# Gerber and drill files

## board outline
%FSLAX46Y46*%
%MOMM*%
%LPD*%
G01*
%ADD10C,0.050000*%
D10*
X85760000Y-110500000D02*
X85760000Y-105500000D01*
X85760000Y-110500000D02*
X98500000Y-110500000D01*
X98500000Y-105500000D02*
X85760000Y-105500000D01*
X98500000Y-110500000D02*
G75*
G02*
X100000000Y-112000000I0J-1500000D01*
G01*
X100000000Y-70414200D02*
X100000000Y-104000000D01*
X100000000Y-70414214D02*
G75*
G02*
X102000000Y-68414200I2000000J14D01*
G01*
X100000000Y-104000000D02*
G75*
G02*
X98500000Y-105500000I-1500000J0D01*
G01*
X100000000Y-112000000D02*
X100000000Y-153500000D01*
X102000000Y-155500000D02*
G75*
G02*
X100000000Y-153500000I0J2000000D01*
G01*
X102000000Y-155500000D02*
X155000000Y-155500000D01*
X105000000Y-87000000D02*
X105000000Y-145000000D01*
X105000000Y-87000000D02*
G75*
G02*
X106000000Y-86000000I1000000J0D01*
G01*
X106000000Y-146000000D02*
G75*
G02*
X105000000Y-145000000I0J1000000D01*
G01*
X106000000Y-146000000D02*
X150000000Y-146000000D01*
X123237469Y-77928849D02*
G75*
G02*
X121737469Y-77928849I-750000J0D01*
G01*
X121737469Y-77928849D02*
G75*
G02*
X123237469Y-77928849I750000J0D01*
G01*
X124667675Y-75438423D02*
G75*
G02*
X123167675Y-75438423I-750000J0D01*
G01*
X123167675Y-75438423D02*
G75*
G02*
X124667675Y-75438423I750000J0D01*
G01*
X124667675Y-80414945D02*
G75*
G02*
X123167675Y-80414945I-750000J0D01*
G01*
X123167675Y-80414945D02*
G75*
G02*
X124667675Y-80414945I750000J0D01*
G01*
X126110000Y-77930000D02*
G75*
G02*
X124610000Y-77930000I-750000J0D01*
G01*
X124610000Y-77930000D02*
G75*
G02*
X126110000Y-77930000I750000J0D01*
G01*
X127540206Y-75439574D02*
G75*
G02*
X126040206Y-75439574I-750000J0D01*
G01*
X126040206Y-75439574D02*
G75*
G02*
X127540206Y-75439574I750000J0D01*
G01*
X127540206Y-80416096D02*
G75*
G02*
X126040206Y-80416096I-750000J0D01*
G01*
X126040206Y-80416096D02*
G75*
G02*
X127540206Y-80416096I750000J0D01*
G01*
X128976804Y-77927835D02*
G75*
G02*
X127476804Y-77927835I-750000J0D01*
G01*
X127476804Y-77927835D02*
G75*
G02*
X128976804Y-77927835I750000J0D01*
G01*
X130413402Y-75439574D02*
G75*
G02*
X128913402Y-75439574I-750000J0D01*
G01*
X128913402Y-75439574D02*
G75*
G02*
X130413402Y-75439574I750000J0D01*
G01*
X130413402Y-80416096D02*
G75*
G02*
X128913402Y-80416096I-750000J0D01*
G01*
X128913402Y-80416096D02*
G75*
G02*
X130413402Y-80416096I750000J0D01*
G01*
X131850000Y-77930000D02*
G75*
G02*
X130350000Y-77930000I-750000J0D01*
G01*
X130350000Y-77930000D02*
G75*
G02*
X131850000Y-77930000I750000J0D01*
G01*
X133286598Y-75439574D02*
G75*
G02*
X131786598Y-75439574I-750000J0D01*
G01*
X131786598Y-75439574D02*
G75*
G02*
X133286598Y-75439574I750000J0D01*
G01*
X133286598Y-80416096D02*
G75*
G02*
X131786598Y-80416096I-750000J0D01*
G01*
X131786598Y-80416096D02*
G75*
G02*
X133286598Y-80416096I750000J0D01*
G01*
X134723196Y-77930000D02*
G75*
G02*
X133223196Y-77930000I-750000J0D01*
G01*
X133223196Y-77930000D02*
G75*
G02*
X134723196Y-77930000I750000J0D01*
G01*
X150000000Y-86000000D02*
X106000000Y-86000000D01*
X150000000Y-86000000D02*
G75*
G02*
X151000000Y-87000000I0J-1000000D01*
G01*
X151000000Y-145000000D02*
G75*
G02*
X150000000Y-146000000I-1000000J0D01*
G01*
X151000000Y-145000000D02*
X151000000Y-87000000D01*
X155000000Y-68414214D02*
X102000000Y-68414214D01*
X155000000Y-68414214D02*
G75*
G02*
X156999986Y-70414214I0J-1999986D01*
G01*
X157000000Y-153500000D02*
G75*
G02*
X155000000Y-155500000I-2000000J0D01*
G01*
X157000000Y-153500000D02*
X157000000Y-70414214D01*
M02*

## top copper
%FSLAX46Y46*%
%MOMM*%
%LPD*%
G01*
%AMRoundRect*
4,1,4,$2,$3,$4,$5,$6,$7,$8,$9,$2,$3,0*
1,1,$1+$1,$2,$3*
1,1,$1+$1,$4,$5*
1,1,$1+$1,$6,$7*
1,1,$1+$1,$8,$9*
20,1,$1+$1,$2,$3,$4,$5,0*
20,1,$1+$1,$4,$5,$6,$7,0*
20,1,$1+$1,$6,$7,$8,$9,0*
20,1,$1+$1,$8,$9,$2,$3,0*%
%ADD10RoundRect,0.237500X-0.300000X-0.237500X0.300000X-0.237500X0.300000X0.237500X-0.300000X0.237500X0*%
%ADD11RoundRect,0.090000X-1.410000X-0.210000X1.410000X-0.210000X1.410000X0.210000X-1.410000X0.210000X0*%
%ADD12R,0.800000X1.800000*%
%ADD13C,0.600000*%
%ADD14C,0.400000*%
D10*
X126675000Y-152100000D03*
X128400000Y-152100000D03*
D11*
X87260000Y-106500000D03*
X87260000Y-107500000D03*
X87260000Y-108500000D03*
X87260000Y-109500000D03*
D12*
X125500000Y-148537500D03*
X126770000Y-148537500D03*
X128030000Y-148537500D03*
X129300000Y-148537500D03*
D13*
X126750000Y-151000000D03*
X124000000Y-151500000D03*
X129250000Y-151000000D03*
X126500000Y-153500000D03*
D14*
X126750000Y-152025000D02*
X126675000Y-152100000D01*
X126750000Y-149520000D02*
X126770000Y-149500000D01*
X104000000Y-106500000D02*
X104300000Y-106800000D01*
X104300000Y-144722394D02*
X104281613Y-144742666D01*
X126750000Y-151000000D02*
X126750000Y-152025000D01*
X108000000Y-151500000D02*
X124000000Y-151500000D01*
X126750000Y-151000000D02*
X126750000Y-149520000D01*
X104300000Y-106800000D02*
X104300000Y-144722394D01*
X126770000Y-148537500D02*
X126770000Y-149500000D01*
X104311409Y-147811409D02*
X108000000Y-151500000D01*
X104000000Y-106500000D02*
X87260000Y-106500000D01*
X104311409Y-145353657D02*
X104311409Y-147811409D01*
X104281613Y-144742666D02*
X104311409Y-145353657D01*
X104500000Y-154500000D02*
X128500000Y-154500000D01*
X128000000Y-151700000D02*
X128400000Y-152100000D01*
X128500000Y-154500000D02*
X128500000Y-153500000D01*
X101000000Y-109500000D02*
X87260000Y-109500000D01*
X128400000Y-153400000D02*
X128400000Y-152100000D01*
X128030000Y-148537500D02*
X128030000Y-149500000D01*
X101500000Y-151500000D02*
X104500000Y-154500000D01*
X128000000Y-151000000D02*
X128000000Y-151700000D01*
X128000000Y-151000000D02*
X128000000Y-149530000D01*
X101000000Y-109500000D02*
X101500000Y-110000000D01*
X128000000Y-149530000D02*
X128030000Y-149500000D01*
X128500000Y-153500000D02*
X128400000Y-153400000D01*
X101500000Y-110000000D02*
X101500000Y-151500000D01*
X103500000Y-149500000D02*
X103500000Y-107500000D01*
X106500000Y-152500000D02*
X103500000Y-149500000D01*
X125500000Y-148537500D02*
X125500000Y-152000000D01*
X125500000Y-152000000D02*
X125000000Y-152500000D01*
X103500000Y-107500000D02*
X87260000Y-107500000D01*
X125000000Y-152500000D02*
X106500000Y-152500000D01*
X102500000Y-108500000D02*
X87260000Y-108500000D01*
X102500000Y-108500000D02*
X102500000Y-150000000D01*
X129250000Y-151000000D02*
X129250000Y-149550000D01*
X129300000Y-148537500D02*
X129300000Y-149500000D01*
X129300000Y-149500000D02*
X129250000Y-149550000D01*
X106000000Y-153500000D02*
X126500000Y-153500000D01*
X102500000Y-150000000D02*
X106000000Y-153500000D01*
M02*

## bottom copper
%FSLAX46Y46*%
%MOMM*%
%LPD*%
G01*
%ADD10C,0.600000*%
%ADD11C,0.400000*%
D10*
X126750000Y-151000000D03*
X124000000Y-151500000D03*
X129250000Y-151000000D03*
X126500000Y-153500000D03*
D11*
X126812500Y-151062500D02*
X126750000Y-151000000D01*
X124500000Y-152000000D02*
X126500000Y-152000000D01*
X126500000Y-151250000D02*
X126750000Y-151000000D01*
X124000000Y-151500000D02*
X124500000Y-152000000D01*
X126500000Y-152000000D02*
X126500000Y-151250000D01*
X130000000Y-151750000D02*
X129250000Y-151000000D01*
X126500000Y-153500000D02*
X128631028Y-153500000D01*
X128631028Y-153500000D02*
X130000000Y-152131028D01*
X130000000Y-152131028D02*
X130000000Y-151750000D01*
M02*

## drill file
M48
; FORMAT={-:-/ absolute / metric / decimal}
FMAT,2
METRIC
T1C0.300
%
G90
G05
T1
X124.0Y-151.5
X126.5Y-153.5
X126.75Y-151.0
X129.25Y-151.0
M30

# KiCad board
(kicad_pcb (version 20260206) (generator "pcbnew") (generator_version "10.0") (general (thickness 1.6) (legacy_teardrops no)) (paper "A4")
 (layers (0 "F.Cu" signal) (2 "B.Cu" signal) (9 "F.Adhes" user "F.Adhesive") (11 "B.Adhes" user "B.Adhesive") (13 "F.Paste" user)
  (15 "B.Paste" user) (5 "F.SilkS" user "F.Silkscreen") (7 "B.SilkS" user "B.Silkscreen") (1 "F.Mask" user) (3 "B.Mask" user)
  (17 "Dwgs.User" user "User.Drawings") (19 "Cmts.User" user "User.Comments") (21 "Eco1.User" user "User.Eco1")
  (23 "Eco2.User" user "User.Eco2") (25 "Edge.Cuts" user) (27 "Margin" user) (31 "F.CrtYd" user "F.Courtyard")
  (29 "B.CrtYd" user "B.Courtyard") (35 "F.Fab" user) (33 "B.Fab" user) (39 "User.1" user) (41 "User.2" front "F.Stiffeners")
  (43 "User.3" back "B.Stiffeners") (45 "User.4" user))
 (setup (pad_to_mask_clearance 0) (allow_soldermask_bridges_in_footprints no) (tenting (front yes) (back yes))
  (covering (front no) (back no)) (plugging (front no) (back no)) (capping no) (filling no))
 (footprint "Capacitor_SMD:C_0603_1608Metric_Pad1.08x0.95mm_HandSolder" (layer "F.Cu") (at 127.5375 152.1)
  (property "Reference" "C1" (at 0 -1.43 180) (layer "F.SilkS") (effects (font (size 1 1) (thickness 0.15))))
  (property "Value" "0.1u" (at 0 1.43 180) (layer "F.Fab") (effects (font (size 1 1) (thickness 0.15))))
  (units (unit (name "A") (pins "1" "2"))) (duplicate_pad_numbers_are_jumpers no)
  (pad "1" smd roundrect (at -0.8625 0) (size 1.075 0.95) (layers "F.Cu" "F.Mask" "F.Paste") (roundrect_rratio 0.25) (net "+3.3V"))
  (pad "2" smd roundrect (at 0.8625 0) (size 1.075 0.95) (layers "F.Cu" "F.Mask" "F.Paste") (roundrect_rratio 0.25) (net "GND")))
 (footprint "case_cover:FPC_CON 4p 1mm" (layer "F.Cu") (at 87.26 108)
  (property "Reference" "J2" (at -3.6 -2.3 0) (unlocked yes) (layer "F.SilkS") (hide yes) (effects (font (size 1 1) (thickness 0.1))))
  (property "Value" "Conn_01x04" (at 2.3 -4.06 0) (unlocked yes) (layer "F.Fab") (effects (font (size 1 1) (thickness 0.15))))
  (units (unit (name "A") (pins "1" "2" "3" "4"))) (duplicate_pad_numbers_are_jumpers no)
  (pad "1" smd roundrect (at 0 -1.5) (size 3 0.6) (layers "F.Cu" "F.Mask" "F.Paste") (roundrect_rratio 0.15) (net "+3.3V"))
  (pad "2" smd roundrect (at 0 -0.5) (size 3 0.6) (layers "F.Cu" "F.Mask" "F.Paste") (roundrect_rratio 0.15) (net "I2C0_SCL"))
  (pad "3" smd roundrect (at 0 0.5) (size 3 0.6) (layers "F.Cu" "F.Mask" "F.Paste") (roundrect_rratio 0.15) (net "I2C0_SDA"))
  (pad "4" smd roundrect (at 0 1.5) (size 3 0.6) (layers "F.Cu" "F.Mask" "F.Paste") (roundrect_rratio 0.15) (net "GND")))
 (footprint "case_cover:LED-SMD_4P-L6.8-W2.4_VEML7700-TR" (layer "F.Cu") (at 127.4 148.5375)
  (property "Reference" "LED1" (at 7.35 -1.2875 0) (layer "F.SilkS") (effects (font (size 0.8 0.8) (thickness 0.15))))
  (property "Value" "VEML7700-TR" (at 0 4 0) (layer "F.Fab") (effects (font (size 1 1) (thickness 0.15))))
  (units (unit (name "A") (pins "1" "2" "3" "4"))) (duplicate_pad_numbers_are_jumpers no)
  (pad "1" smd rect (at -1.9 0) (size 0.8 1.8) (layers "F.Cu" "F.Mask" "F.Paste") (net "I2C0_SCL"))
  (pad "2" smd rect (at -0.63 0) (size 0.8 1.8) (layers "F.Cu" "F.Mask" "F.Paste") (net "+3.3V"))
  (pad "3" smd rect (at 0.63 0) (size 0.8 1.8) (layers "F.Cu" "F.Mask" "F.Paste") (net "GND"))
  (pad "4" smd rect (at 1.9 0) (size 0.8 1.8) (layers "F.Cu" "F.Mask" "F.Paste") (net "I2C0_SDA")))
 (gr_line (start 85.76 110.5) (end 85.76 105.5) (stroke (width 0.05) (type default)) (layer "Edge.Cuts"))
 (gr_line (start 85.76 110.5) (end 98.5 110.5) (stroke (width 0.05) (type default)) (layer "Edge.Cuts"))
 (gr_line (start 98.5 105.5) (end 85.76 105.5) (stroke (width 0.05) (type default)) (layer "Edge.Cuts"))
 (gr_arc (start 98.5 110.5) (mid 99.56066 110.93934) (end 100 112) (stroke (width 0.05) (type default)) (layer "Edge.Cuts"))
 (gr_line (start 100 70.4142) (end 100 104) (stroke (width 0.05) (type default)) (layer "Edge.Cuts"))
 (gr_arc (start 100 70.414214) (mid 100.585786 69) (end 102 68.414214) (stroke (width 0.05) (type default)) (layer "Edge.Cuts"))
 (gr_arc (start 100 104) (mid 99.56066 105.06066) (end 98.5 105.5) (stroke (width 0.05) (type default)) (layer "Edge.Cuts"))
 (gr_line (start 100 112) (end 100 153.5) (stroke (width 0.05) (type default)) (layer "Edge.Cuts"))
 (gr_arc (start 102 155.5) (mid 100.585786 154.914214) (end 100 153.5) (stroke (width 0.05) (type default)) (layer "Edge.Cuts"))
 (gr_line (start 102 155.5) (end 155 155.5) (stroke (width 0.05) (type default)) (layer "Edge.Cuts"))
 (gr_line (start 105 87) (end 105 145) (stroke (width 0.05) (type default)) (layer "Edge.Cuts"))
 (gr_arc (start 105 87) (mid 105.292893 86.292893) (end 106 86) (stroke (width 0.05) (type default)) (layer "Edge.Cuts"))
 (gr_arc (start 106 146) (mid 105.292893 145.707107) (end 105 145) (stroke (width 0.05) (type default)) (layer "Edge.Cuts"))
 (gr_line (start 106 146) (end 150 146) (stroke (width 0.05) (type default)) (layer "Edge.Cuts"))
 (gr_circle (center 122.487469 77.928849) (end 123.237469 77.928849) (stroke (width 0.05) (type solid)) (fill no) (layer "Edge.Cuts"))
 (gr_circle (center 123.917675 75.438423) (end 124.667675 75.438423) (stroke (width 0.05) (type solid)) (fill no) (layer "Edge.Cuts"))
 (gr_circle (center 123.917675 80.414945) (end 124.667675 80.414945) (stroke (width 0.05) (type solid)) (fill no) (layer "Edge.Cuts"))
 (gr_circle (center 125.36 77.93) (end 126.11 77.93) (stroke (width 0.05) (type solid)) (fill no) (layer "Edge.Cuts"))
 (gr_circle (center 126.790206 75.439574) (end 127.540206 75.439574) (stroke (width 0.05) (type solid)) (fill no) (layer "Edge.Cuts"))
 (gr_circle (center 126.790206 80.416096) (end 127.540206 80.416096) (stroke (width 0.05) (type solid)) (fill no) (layer "Edge.Cuts"))
 (gr_circle (center 128.226804 77.927835) (end 128.976804 77.927835) (stroke (width 0.05) (type solid)) (fill no) (layer "Edge.Cuts"))
 (gr_circle (center 129.663402 75.439574) (end 130.413402 75.439574) (stroke (width 0.05) (type solid)) (fill no) (layer "Edge.Cuts"))
 (gr_circle (center 129.663402 80.416096) (end 130.413402 80.416096) (stroke (width 0.05) (type solid)) (fill no) (layer "Edge.Cuts"))
 (gr_circle (center 131.1 77.93) (end 131.85 77.93) (stroke (width 0.05) (type solid)) (fill no) (layer "Edge.Cuts"))
 (gr_circle (center 132.536598 75.439574) (end 133.286598 75.439574) (stroke (width 0.05) (type solid)) (fill no) (layer "Edge.Cuts"))
 (gr_circle (center 132.536598 80.416096) (end 133.286598 80.416096) (stroke (width 0.05) (type solid)) (fill no) (layer "Edge.Cuts"))
 (gr_circle (center 133.973196 77.93) (end 134.723196 77.93) (stroke (width 0.05) (type solid)) (fill no) (layer "Edge.Cuts"))
 (gr_line (start 150 86) (end 106 86) (stroke (width 0.05) (type default)) (layer "Edge.Cuts"))
 (gr_arc (start 150 86) (mid 150.707107 86.292893) (end 151 87) (stroke (width 0.05) (type default)) (layer "Edge.Cuts"))
 (gr_arc (start 151 145) (mid 150.707107 145.707107) (end 150 146) (stroke (width 0.05) (type default)) (layer "Edge.Cuts"))
 (gr_line (start 151 145) (end 151 87) (stroke (width 0.05) (type default)) (layer "Edge.Cuts"))
 (gr_line (start 155 68.414214) (end 102 68.414214) (stroke (width 0.05) (type default)) (layer "Edge.Cuts"))
 (gr_arc (start 155 68.414214) (mid 156.414214 69) (end 157 70.414214) (stroke (width 0.05) (type default)) (layer "Edge.Cuts"))
 (gr_arc (start 157 153.5) (mid 156.414214 154.914214) (end 155 155.5) (stroke (width 0.05) (type default)) (layer "Edge.Cuts"))
 (gr_line (start 157 153.5) (end 157 70.414214) (stroke (width 0.05) (type default)) (layer "Edge.Cuts"))
 (segment (start 126.75 152.025) (end 126.675 152.1) (width 0.4) (layer "F.Cu") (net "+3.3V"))
 (segment (start 126.75 149.52) (end 126.77 149.5) (width 0.4) (layer "F.Cu") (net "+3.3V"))
 (segment (start 104 106.5) (end 104.3 106.8) (width 0.4) (layer "F.Cu") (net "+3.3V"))
 (segment (start 104.3 144.722394) (end 104.281613 144.742666) (width 0.4) (layer "F.Cu") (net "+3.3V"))
 (segment (start 126.75 151) (end 126.75 152.025) (width 0.4) (layer "F.Cu") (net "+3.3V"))
 (segment (start 108 151.5) (end 124 151.5) (width 0.4) (layer "F.Cu") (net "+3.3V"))
 (segment (start 126.75 151) (end 126.75 149.52) (width 0.4) (layer "F.Cu") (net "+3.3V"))
 (segment (start 104.3 106.8) (end 104.3 144.722394) (width 0.4) (layer "F.Cu") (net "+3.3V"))
 (segment (start 126.77 148.5375) (end 126.77 149.5) (width 0.4) (layer "F.Cu") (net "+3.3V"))
 (segment (start 104.311409 147.811409) (end 108 151.5) (width 0.4) (layer "F.Cu") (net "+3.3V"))
 (segment (start 104 106.5) (end 87.26 106.5) (width 0.4) (layer "F.Cu") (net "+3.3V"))
 (segment (start 104.311409 145.353657) (end 104.311409 147.811409) (width 0.4) (layer "F.Cu") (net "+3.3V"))
 (segment (start 104.281613 144.742666) (end 104.311409 145.353657) (width 0.4) (layer "F.Cu") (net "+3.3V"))
 (via (at 126.75 151) (size 0.6) (drill 0.3) (layers "F.Cu" "B.Cu") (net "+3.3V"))
 (via (at 124 151.5) (size 0.6) (drill 0.3) (layers "F.Cu" "B.Cu") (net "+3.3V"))
 (segment (start 126.8125 151.0625) (end 126.75 151) (width 0.4) (layer "B.Cu") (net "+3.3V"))
 (segment (start 124.5 152) (end 126.5 152) (width 0.4) (layer "B.Cu") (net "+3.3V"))
 (segment (start 126.5 151.25) (end 126.75 151) (width 0.4) (layer "B.Cu") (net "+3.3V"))
 (segment (start 124 151.5) (end 124.5 152) (width 0.4) (layer "B.Cu") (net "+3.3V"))
 (segment (start 126.5 152) (end 126.5 151.25) (width 0.4) (layer "B.Cu") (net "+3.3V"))
 (segment (start 104.5 154.5) (end 128.5 154.5) (width 0.4) (layer "F.Cu") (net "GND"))
 (segment (start 128 151.7) (end 128.4 152.1) (width 0.4) (layer "F.Cu") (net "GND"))
 (segment (start 128.5 154.5) (end 128.5 153.5) (width 0.4) (layer "F.Cu") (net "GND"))
 (segment (start 101 109.5) (end 87.26 109.5) (width 0.4) (layer "F.Cu") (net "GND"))
 (segment (start 128.4 153.4) (end 128.4 152.1) (width 0.4) (layer "F.Cu") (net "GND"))
 (segment (start 128.03 148.5375) (end 128.03 149.5) (width 0.4) (layer "F.Cu") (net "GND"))
 (segment (start 101.5 151.5) (end 104.5 154.5) (width 0.4) (layer "F.Cu") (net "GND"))
 (segment (start 128 151) (end 128 151.7) (width 0.4) (layer "F.Cu") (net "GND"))
 (segment (start 128 151) (end 128 149.53) (width 0.4) (layer "F.Cu") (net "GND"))
 (segment (start 101 109.5) (end 101.5 110) (width 0.4) (layer "F.Cu") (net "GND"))
 (segment (start 128 149.53) (end 128.03 149.5) (width 0.4) (layer "F.Cu") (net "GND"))
 (segment (start 128.5 153.5) (end 128.4 153.4) (width 0.4) (layer "F.Cu") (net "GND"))
 (segment (start 101.5 110) (end 101.5 151.5) (width 0.4) (layer "F.Cu") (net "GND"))
 (segment (start 103.5 149.5) (end 103.5 107.5) (width 0.4) (layer "F.Cu") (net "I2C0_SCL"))
 (segment (start 106.5 152.5) (end 103.5 149.5) (width 0.4) (layer "F.Cu") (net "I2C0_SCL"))
 (segment (start 125.5 148.5375) (end 125.5 152) (width 0.4) (layer "F.Cu") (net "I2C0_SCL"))
 (segment (start 125.5 152) (end 125 152.5) (width 0.4) (layer "F.Cu") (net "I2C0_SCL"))
 (segment (start 103.5 107.5) (end 87.26 107.5) (width 0.4) (layer "F.Cu") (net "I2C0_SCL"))
 (segment (start 125 152.5) (end 106.5 152.5) (width 0.4) (layer "F.Cu") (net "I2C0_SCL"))
 (segment (start 102.5 108.5) (end 87.26 108.5) (width 0.4) (layer "F.Cu") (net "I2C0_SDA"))
 (segment (start 102.5 108.5) (end 102.5 150) (width 0.4) (layer "F.Cu") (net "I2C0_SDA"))
 (segment (start 129.25 151) (end 129.25 149.55) (width 0.4) (layer "F.Cu") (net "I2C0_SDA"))
 (segment (start 129.3 148.5375) (end 129.3 149.5) (width 0.4) (layer "F.Cu") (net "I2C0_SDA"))
 (segment (start 129.3 149.5) (end 129.25 149.55) (width 0.4) (layer "F.Cu") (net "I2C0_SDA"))
 (segment (start 106 153.5) (end 126.5 153.5) (width 0.4) (layer "F.Cu") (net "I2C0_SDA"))
 (segment (start 102.5 150) (end 106 153.5) (width 0.4) (layer "F.Cu") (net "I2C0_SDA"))
 (via (at 129.25 151) (size 0.6) (drill 0.3) (layers "F.Cu" "B.Cu") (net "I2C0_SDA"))
 (via (at 126.5 153.5) (size 0.6) (drill 0.3) (layers "F.Cu" "B.Cu") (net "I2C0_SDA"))
 (segment (start 130 151.75) (end 129.25 151) (width 0.4) (layer "B.Cu") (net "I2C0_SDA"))
 (segment (start 126.5 153.5) (end 128.631028 153.5) (width 0.4) (layer "B.Cu") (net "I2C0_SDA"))
 (segment (start 128.631028 153.5) (end 130 152.131028) (width 0.4) (layer "B.Cu") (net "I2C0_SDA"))
 (segment (start 130 152.131028) (end 130 151.75) (width 0.4) (layer "B.Cu") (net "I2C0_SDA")))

